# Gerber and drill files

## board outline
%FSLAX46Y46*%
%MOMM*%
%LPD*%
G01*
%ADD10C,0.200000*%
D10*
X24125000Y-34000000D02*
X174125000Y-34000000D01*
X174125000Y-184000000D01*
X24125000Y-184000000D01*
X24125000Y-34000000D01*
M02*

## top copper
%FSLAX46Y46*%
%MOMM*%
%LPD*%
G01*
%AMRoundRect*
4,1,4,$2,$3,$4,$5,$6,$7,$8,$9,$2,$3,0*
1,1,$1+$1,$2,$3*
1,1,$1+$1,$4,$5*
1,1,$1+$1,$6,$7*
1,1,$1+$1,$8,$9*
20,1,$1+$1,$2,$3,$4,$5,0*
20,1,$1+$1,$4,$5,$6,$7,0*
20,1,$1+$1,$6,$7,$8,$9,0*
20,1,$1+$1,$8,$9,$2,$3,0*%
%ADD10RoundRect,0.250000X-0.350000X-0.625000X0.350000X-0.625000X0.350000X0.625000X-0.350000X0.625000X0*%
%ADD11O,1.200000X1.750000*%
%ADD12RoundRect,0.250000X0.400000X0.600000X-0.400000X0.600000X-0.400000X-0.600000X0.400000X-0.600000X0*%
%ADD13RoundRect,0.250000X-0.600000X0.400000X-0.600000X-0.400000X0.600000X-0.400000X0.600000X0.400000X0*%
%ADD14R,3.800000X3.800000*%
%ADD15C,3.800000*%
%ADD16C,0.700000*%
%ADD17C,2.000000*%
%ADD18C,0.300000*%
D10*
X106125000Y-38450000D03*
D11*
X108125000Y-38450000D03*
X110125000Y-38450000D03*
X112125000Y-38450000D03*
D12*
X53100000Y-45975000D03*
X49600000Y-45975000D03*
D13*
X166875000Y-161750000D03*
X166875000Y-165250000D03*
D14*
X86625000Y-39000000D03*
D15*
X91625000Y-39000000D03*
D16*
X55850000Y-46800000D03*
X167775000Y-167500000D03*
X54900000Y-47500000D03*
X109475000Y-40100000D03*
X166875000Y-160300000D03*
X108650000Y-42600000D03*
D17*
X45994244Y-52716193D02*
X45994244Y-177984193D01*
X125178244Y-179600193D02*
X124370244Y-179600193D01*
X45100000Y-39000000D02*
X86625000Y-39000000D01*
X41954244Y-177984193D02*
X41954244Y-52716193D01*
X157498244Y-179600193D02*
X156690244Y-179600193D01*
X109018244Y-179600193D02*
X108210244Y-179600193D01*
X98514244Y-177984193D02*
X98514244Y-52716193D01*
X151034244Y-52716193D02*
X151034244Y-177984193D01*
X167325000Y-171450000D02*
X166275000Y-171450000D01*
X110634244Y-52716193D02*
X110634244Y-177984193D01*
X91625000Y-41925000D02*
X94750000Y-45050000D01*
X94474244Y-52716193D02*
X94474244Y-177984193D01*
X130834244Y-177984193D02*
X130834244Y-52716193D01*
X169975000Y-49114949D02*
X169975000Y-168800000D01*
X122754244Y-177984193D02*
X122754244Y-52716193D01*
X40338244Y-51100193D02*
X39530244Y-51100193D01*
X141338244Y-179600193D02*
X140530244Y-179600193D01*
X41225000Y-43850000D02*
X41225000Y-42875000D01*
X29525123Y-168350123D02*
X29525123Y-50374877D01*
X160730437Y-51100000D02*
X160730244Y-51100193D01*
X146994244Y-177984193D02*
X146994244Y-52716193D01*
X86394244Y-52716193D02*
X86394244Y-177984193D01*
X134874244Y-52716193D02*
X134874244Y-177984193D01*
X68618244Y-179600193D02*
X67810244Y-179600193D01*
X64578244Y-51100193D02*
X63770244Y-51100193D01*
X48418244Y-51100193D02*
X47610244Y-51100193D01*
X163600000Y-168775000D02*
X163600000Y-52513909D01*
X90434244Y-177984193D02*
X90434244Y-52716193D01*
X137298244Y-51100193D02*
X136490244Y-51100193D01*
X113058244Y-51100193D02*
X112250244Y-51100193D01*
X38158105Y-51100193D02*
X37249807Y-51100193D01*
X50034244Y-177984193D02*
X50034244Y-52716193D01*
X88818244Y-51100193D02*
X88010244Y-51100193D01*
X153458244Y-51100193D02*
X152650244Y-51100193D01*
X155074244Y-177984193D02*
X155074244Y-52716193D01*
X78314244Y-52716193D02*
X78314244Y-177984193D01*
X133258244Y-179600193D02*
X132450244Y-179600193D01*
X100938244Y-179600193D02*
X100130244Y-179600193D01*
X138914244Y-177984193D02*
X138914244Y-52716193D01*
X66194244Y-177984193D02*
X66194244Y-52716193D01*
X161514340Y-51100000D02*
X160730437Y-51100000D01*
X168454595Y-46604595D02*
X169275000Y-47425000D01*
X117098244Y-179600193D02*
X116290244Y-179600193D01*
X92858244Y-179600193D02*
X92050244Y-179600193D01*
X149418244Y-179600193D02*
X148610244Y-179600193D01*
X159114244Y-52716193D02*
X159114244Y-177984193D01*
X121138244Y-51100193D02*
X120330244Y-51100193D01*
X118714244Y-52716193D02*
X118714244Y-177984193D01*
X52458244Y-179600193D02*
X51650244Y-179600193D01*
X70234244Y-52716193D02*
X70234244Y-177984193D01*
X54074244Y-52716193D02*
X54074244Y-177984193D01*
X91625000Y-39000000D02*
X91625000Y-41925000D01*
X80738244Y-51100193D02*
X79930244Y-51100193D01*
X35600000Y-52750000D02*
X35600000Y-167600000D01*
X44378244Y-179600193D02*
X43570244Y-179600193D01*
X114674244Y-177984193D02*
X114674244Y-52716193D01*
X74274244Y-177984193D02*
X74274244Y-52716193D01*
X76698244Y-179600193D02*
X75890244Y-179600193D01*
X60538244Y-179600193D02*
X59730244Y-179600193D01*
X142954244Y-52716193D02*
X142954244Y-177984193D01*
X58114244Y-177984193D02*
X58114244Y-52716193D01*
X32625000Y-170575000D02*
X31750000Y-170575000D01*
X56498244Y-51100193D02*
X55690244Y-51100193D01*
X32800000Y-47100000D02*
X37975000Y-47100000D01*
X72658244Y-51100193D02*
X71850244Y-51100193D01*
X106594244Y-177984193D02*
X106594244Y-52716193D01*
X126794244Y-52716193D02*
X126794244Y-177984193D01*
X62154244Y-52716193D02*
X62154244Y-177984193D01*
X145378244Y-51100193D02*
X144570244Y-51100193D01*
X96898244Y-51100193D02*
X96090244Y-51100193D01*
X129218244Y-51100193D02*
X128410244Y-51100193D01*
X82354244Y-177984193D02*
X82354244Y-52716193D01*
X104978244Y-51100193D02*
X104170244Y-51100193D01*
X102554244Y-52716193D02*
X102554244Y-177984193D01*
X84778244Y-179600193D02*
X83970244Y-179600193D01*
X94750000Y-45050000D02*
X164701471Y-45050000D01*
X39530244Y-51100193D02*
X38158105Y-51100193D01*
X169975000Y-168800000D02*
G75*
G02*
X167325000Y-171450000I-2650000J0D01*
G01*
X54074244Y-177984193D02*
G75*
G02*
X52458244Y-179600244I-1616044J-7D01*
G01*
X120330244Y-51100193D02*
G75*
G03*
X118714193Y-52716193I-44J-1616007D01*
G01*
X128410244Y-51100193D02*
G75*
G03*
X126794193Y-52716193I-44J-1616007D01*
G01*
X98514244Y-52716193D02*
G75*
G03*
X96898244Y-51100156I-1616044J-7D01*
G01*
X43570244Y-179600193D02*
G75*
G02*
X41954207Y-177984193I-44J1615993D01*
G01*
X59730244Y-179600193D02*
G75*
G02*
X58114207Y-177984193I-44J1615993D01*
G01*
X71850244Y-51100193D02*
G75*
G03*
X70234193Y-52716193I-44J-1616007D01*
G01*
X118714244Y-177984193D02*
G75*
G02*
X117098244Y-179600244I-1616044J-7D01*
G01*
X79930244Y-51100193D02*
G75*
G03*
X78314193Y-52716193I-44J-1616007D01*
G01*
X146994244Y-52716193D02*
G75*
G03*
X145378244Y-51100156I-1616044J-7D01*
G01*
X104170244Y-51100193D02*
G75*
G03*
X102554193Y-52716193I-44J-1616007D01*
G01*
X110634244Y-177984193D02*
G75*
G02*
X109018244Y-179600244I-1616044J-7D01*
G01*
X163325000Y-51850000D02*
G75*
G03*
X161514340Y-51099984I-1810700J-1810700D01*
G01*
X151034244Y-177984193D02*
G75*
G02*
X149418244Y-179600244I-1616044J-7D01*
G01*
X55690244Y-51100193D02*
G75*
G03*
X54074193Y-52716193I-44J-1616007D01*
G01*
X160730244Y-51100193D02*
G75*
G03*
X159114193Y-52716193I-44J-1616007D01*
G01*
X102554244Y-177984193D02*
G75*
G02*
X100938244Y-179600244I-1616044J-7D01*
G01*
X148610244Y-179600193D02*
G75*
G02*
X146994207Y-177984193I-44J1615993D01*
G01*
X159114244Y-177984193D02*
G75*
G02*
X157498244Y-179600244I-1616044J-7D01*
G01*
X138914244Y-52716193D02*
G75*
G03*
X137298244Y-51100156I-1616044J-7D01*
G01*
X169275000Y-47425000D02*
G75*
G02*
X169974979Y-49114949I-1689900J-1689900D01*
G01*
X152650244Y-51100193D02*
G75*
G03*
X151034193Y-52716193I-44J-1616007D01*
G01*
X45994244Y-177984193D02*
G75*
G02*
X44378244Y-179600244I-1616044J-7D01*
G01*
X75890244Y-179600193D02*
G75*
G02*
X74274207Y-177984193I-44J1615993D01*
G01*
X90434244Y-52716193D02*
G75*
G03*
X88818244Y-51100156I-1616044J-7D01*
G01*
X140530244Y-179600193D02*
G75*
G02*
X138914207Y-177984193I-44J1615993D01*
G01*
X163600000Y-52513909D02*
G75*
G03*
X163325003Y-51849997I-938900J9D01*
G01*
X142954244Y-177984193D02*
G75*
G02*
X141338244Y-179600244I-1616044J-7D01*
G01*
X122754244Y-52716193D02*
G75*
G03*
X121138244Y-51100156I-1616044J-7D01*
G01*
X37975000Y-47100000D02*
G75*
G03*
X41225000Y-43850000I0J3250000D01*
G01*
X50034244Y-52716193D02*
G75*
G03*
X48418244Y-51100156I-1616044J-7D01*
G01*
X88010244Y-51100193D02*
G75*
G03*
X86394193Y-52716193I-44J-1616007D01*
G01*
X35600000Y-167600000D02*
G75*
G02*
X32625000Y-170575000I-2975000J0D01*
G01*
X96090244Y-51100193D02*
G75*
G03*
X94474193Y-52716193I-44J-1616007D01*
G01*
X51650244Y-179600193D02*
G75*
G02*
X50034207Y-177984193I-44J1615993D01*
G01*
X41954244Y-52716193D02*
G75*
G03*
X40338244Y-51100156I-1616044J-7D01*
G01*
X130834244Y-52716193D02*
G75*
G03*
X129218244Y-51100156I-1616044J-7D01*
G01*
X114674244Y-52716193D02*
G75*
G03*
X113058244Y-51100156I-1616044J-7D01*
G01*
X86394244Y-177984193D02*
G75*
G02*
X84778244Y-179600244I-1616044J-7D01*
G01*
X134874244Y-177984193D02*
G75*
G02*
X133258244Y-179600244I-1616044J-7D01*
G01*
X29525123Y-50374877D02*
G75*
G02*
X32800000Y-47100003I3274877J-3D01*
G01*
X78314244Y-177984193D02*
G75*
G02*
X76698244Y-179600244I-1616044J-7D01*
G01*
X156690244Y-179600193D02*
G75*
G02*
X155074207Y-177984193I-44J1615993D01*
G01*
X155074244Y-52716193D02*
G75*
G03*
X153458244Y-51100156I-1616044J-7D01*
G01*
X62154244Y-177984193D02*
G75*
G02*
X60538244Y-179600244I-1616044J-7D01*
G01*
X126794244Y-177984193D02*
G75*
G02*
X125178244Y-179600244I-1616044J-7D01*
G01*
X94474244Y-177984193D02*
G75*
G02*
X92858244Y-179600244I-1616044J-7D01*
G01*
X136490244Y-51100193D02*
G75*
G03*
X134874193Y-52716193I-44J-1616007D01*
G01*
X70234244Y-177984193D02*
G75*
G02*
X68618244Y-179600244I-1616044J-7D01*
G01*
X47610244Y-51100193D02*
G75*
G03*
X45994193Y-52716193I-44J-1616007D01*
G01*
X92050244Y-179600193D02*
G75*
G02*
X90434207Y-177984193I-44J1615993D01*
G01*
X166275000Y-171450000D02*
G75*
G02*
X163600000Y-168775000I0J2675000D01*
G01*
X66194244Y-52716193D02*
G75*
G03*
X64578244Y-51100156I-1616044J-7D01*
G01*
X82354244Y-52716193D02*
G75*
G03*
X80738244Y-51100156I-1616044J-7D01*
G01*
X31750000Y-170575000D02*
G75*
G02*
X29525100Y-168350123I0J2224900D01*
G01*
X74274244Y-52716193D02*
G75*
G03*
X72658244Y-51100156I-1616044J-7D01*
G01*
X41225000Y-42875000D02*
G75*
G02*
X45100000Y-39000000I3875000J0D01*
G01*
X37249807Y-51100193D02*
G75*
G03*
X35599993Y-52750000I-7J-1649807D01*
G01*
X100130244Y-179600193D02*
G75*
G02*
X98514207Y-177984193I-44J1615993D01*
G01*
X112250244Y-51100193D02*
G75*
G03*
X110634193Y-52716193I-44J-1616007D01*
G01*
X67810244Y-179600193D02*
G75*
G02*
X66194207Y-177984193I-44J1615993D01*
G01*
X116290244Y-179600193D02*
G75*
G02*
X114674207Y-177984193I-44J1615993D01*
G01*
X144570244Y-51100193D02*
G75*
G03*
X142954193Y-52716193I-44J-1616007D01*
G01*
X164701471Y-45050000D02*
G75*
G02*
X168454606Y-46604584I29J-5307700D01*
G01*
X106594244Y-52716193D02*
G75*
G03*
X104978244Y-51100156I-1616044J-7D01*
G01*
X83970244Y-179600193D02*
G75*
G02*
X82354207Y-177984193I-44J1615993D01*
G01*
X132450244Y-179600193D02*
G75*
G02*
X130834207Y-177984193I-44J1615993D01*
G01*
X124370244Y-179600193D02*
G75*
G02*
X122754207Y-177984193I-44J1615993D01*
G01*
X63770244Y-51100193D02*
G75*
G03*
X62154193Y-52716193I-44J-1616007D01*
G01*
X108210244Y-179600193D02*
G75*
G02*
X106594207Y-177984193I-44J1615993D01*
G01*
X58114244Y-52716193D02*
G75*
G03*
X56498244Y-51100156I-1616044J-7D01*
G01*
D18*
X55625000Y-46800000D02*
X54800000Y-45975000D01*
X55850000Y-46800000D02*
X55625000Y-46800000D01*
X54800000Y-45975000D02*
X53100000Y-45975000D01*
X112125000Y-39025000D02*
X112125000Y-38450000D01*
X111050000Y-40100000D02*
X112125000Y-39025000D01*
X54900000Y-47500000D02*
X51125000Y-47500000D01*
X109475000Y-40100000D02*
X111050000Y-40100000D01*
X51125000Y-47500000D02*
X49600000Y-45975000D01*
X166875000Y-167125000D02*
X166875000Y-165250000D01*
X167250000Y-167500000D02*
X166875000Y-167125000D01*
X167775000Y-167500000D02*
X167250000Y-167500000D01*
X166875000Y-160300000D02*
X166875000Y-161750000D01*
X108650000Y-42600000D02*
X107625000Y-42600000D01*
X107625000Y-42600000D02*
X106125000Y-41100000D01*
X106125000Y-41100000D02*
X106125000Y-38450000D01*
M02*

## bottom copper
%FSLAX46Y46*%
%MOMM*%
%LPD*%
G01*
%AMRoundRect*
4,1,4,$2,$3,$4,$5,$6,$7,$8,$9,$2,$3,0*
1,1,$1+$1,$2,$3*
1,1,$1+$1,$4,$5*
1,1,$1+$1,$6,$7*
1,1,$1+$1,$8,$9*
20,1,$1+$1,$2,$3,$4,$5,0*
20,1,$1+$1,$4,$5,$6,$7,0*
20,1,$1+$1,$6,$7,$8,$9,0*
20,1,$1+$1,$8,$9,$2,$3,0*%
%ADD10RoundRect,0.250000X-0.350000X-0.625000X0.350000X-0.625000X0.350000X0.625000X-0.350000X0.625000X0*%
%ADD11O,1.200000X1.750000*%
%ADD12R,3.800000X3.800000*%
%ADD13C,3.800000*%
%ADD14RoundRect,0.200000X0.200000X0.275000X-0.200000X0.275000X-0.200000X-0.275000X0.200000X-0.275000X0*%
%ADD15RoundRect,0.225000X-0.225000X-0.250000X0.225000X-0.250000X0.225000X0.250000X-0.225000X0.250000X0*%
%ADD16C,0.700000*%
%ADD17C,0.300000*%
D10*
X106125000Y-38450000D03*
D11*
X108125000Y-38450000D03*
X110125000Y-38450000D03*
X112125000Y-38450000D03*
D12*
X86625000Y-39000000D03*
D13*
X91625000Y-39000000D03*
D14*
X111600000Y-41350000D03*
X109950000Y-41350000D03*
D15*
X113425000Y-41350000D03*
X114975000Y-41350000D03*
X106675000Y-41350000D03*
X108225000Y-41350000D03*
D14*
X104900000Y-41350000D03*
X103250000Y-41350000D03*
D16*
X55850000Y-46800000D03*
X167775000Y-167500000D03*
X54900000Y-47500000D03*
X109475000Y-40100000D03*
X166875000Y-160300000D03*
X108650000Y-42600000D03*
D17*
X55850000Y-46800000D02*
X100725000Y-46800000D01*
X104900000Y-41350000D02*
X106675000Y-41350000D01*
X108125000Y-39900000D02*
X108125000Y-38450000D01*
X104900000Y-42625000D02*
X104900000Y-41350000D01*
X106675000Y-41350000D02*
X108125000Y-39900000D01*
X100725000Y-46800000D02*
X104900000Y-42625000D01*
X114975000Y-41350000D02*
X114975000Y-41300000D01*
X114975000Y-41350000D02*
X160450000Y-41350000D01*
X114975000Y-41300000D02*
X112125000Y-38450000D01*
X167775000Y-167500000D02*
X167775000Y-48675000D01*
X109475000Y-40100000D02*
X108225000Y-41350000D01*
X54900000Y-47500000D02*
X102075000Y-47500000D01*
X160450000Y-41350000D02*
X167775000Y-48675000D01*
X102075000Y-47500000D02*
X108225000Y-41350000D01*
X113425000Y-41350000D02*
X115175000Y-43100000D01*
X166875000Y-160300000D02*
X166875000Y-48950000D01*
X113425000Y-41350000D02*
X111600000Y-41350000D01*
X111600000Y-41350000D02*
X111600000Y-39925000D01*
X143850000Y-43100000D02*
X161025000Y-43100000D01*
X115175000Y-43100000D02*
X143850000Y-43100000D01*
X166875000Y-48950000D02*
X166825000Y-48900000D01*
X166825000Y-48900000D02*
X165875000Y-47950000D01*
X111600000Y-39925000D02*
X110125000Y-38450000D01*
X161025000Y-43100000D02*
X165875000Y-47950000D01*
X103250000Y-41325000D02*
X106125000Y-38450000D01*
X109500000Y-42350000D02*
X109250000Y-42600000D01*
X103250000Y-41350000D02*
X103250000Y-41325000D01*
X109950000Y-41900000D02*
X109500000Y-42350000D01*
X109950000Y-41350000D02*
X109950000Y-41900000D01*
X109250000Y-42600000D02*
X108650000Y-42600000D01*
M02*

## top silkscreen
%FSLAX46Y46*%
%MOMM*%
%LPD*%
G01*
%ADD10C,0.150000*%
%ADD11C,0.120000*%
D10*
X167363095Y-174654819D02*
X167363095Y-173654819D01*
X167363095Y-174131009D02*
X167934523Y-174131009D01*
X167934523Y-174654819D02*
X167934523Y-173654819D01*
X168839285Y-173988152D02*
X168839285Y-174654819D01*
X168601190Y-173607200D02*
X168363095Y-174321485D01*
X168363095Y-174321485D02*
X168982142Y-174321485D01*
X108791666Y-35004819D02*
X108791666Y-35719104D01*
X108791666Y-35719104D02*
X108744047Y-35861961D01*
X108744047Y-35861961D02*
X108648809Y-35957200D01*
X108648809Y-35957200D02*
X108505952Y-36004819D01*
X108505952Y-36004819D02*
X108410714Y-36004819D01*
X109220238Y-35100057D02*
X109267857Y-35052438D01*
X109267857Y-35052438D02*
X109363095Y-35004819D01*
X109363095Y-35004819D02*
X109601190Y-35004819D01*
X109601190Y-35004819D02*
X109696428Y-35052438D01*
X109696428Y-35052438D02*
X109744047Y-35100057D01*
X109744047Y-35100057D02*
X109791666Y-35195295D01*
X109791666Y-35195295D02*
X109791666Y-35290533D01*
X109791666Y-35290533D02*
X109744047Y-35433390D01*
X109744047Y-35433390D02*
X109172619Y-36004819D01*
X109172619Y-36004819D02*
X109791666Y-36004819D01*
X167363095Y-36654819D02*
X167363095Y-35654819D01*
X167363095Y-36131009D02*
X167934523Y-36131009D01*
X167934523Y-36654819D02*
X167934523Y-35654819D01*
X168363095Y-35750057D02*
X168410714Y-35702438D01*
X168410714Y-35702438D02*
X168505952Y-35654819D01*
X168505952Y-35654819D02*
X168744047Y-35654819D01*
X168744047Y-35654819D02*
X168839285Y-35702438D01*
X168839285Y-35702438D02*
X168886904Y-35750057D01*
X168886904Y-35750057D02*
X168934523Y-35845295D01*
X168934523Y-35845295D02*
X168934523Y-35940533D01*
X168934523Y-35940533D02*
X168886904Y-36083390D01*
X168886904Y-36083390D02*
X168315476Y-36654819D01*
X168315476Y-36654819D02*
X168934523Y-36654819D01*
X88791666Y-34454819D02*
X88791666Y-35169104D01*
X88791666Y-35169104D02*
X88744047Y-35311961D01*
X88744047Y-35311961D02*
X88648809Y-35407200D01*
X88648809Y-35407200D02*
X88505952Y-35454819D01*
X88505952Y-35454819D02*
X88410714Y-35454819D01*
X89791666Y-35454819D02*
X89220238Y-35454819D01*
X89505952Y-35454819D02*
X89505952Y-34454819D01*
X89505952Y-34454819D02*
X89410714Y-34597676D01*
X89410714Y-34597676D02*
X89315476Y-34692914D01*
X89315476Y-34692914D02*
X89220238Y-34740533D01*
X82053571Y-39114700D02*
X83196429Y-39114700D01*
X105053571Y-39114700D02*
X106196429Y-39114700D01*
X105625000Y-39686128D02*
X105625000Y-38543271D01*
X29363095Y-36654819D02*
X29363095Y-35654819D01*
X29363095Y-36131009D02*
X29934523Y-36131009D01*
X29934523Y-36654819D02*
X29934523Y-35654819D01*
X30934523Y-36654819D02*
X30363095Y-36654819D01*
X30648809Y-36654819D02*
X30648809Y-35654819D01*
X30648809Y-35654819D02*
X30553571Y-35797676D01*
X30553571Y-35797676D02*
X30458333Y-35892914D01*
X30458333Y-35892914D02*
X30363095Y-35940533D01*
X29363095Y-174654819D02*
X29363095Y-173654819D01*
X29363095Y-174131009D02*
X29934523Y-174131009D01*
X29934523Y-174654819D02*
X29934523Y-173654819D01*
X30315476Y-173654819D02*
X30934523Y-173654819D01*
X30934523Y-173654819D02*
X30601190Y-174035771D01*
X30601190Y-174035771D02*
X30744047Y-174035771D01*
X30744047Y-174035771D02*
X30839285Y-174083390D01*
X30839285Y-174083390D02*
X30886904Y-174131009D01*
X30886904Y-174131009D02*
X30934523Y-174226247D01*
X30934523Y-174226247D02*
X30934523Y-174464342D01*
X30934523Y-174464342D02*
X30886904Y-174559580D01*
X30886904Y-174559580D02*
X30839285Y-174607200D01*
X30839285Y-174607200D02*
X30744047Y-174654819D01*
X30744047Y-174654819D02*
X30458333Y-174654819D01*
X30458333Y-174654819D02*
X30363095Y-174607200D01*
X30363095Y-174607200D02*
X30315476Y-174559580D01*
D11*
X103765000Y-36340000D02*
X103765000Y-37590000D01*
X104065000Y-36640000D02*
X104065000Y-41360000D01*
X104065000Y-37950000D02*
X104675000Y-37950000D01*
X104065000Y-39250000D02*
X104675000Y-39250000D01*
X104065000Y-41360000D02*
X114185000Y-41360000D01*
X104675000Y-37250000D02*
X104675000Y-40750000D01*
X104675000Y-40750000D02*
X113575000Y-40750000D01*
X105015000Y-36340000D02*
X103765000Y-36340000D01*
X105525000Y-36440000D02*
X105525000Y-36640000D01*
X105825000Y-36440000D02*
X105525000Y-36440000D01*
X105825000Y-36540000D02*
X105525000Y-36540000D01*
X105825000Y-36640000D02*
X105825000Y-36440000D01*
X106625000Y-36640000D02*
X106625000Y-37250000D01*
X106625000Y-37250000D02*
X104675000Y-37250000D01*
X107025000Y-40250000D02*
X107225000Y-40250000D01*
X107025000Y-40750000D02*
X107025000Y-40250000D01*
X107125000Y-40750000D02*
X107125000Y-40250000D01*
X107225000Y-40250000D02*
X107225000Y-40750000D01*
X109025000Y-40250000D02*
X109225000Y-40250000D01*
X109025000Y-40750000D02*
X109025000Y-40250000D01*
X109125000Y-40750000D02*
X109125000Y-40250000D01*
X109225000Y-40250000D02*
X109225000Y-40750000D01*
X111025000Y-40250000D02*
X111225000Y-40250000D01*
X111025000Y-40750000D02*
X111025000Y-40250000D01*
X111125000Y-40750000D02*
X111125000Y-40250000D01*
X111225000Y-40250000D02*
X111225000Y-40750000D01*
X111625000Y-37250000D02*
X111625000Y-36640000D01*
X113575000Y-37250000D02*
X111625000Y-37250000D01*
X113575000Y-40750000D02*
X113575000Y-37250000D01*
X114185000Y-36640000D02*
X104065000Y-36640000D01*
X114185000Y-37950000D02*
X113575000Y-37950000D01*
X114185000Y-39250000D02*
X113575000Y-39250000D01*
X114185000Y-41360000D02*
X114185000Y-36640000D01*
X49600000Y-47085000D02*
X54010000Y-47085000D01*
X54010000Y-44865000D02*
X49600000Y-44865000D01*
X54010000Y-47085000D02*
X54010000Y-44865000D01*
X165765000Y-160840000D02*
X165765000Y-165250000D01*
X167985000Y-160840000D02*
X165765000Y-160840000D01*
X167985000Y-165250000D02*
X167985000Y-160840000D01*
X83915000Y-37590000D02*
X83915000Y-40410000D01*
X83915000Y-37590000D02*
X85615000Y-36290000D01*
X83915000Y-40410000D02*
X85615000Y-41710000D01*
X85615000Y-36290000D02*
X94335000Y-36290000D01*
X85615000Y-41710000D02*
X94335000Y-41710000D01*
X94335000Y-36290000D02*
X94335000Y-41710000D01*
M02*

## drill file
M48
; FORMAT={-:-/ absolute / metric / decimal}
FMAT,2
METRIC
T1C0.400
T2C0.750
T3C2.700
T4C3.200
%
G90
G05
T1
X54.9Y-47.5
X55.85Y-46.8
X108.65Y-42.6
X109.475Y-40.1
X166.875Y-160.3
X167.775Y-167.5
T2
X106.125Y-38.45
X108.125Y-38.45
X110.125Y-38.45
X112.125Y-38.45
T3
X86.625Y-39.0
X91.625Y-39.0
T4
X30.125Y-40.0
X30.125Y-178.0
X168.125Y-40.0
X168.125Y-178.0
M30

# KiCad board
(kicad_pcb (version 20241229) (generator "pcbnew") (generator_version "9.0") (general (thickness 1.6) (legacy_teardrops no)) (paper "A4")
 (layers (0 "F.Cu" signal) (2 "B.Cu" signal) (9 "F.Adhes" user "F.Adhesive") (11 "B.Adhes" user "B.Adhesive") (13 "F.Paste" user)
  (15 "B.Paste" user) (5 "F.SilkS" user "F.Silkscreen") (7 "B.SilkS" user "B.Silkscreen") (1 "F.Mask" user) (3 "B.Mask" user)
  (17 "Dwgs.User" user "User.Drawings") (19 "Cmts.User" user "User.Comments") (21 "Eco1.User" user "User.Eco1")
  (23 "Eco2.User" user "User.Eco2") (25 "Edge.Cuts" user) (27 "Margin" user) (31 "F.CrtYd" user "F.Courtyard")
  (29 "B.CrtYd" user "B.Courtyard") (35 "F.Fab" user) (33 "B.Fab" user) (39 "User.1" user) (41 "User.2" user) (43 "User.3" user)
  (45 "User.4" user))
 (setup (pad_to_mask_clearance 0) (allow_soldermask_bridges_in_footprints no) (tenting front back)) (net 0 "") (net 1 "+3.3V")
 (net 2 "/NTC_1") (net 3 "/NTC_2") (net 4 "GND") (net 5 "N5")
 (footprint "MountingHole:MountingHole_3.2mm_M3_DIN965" (layer "F.Cu") (at 168.125 178)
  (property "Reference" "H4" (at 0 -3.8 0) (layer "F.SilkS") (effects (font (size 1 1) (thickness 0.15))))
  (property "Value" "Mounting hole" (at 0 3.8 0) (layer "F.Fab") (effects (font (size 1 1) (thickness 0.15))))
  (pad "" np_thru_hole circle (at 0 0) (size 3.2 3.2) (drill 3.2) (layers "*.Cu" "*.Mask")))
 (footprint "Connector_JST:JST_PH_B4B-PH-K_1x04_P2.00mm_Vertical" (layer "F.Cu") (at 106.125 38.45)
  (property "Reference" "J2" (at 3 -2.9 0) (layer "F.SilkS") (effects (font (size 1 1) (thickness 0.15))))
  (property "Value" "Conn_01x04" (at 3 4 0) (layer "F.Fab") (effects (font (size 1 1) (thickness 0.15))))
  (fp_line (start -2.36 -2.11) (end -2.36 -0.86) (stroke (width 0.12) (type solid)) (layer "F.SilkS"))
  (fp_line (start -2.06 -1.81) (end -2.06 2.91) (stroke (width 0.12) (type solid)) (layer "F.SilkS"))
  (fp_line (start -2.06 -0.5) (end -1.45 -0.5) (stroke (width 0.12) (type solid)) (layer "F.SilkS"))
  (fp_line (start -2.06 0.8) (end -1.45 0.8) (stroke (width 0.12) (type solid)) (layer "F.SilkS"))
  (fp_line (start -2.06 2.91) (end 8.06 2.91) (stroke (width 0.12) (type solid)) (layer "F.SilkS"))
  (fp_line (start -1.45 -1.2) (end -1.45 2.3) (stroke (width 0.12) (type solid)) (layer "F.SilkS"))
  (fp_line (start -1.45 2.3) (end 7.45 2.3) (stroke (width 0.12) (type solid)) (layer "F.SilkS"))
  (fp_line (start -1.11 -2.11) (end -2.36 -2.11) (stroke (width 0.12) (type solid)) (layer "F.SilkS"))
  (fp_line (start -0.6 -2.01) (end -0.6 -1.81) (stroke (width 0.12) (type solid)) (layer "F.SilkS"))
  (fp_line (start -0.3 -2.01) (end -0.6 -2.01) (stroke (width 0.12) (type solid)) (layer "F.SilkS"))
  (fp_line (start -0.3 -1.91) (end -0.6 -1.91) (stroke (width 0.12) (type solid)) (layer "F.SilkS"))
  (fp_line (start -0.3 -1.81) (end -0.3 -2.01) (stroke (width 0.12) (type solid)) (layer "F.SilkS"))
  (fp_line (start 0.5 -1.81) (end 0.5 -1.2) (stroke (width 0.12) (type solid)) (layer "F.SilkS"))
  (fp_line (start 0.5 -1.2) (end -1.45 -1.2) (stroke (width 0.12) (type solid)) (layer "F.SilkS"))
  (fp_line (start 0.9 1.8) (end 1.1 1.8) (stroke (width 0.12) (type solid)) (layer "F.SilkS"))
  (fp_line (start 0.9 2.3) (end 0.9 1.8) (stroke (width 0.12) (type solid)) (layer "F.SilkS"))
  (fp_line (start 1 2.3) (end 1 1.8) (stroke (width 0.12) (type solid)) (layer "F.SilkS"))
  (fp_line (start 1.1 1.8) (end 1.1 2.3) (stroke (width 0.12) (type solid)) (layer "F.SilkS"))
  (fp_line (start 2.9 1.8) (end 3.1 1.8) (stroke (width 0.12) (type solid)) (layer "F.SilkS"))
  (fp_line (start 2.9 2.3) (end 2.9 1.8) (stroke (width 0.12) (type solid)) (layer "F.SilkS"))
  (fp_line (start 3 2.3) (end 3 1.8) (stroke (width 0.12) (type solid)) (layer "F.SilkS"))
  (fp_line (start 3.1 1.8) (end 3.1 2.3) (stroke (width 0.12) (type solid)) (layer "F.SilkS"))
  (fp_line (start 4.9 1.8) (end 5.1 1.8) (stroke (width 0.12) (type solid)) (layer "F.SilkS"))
  (fp_line (start 4.9 2.3) (end 4.9 1.8) (stroke (width 0.12) (type solid)) (layer "F.SilkS"))
  (fp_line (start 5 2.3) (end 5 1.8) (stroke (width 0.12) (type solid)) (layer "F.SilkS"))
  (fp_line (start 5.1 1.8) (end 5.1 2.3) (stroke (width 0.12) (type solid)) (layer "F.SilkS"))
  (fp_line (start 5.5 -1.2) (end 5.5 -1.81) (stroke (width 0.12) (type solid)) (layer "F.SilkS"))
  (fp_line (start 7.45 -1.2) (end 5.5 -1.2) (stroke (width 0.12) (type solid)) (layer "F.SilkS"))
  (fp_line (start 7.45 2.3) (end 7.45 -1.2) (stroke (width 0.12) (type solid)) (layer "F.SilkS"))
  (fp_line (start 8.06 -1.81) (end -2.06 -1.81) (stroke (width 0.12) (type solid)) (layer "F.SilkS"))
  (fp_line (start 8.06 -0.5) (end 7.45 -0.5) (stroke (width 0.12) (type solid)) (layer "F.SilkS"))
  (fp_line (start 8.06 0.8) (end 7.45 0.8) (stroke (width 0.12) (type solid)) (layer "F.SilkS"))
  (fp_line (start 8.06 2.91) (end 8.06 -1.81) (stroke (width 0.12) (type solid)) (layer "F.SilkS"))
  (pad "1" thru_hole roundrect (at 0 0) (size 1.2 1.75) (drill 0.75) (layers "*.Cu" "*.Mask") (remove_unused_layers no)
   (roundrect_rratio 0.208333) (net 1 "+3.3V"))
  (pad "2" thru_hole oval (at 2 0) (size 1.2 1.75) (drill 0.75) (layers "*.Cu" "*.Mask") (remove_unused_layers no) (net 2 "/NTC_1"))
  (pad "3" thru_hole oval (at 4 0) (size 1.2 1.75) (drill 0.75) (layers "*.Cu" "*.Mask") (remove_unused_layers no) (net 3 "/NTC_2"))
  (pad "4" thru_hole oval (at 6 0) (size 1.2 1.75) (drill 0.75) (layers "*.Cu" "*.Mask") (remove_unused_layers no) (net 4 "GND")))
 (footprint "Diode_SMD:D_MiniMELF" (layer "F.Cu") (at 51.35 45.975 180)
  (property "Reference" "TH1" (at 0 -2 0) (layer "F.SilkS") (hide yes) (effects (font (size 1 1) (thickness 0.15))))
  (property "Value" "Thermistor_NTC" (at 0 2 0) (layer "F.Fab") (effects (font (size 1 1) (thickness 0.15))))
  (fp_line (start 1.75 -1.11) (end -2.66 -1.11) (stroke (width 0.12) (type solid)) (layer "F.SilkS"))
  (fp_line (start -2.66 1.11) (end 1.75 1.11) (stroke (width 0.12) (type solid)) (layer "F.SilkS"))
  (fp_line (start -2.66 -1.11) (end -2.66 1.11) (stroke (width 0.12) (type solid)) (layer "F.SilkS"))
  (pad "1" smd roundrect (at -1.75 0 180) (size 1.3 1.7) (layers "F.Cu" "F.Mask" "F.Paste") (roundrect_rratio 0.1923076923) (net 2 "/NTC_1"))
  (pad "2" smd roundrect (at 1.75 0 180) (size 1.3 1.7) (layers "F.Cu" "F.Mask" "F.Paste") (roundrect_rratio 0.1923076923) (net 4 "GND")))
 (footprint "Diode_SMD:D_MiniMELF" (layer "F.Cu") (at 166.875 163.5 -90)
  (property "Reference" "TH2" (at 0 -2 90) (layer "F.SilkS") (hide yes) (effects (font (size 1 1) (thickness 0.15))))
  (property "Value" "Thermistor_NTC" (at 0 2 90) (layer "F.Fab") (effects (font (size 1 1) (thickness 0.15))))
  (fp_line (start -2.66 1.11) (end 1.75 1.11) (stroke (width 0.12) (type solid)) (layer "F.SilkS"))
  (fp_line (start -2.66 -1.11) (end -2.66 1.11) (stroke (width 0.12) (type solid)) (layer "F.SilkS"))
  (fp_line (start 1.75 -1.11) (end -2.66 -1.11) (stroke (width 0.12) (type solid)) (layer "F.SilkS"))
  (pad "1" smd roundrect (at -1.75 0 270) (size 1.3 1.7) (layers "F.Cu" "F.Mask" "F.Paste") (roundrect_rratio 0.1923076923) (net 3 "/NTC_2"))
  (pad "2" smd roundrect (at 1.75 0 270) (size 1.3 1.7) (layers "F.Cu" "F.Mask" "F.Paste") (roundrect_rratio 0.1923076923) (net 4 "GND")))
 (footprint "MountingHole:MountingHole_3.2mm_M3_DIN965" (layer "F.Cu") (at 168.125 40)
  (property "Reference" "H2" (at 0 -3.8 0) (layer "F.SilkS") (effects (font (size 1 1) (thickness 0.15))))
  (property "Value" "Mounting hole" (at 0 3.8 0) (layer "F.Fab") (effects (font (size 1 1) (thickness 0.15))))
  (pad "" np_thru_hole circle (at 0 0) (size 3.2 3.2) (drill 3.2) (layers "*.Cu" "*.Mask")))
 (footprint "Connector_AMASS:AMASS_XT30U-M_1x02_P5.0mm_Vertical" (layer "F.Cu") (at 86.625 39)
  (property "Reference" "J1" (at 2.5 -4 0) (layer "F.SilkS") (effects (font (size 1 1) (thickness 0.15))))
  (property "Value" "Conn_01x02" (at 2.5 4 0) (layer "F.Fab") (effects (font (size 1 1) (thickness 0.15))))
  (fp_line (start -2.71 -1.41) (end -2.71 1.41) (stroke (width 0.12) (type solid)) (layer "F.SilkS"))
  (fp_line (start -2.71 -1.41) (end -1.01 -2.71) (stroke (width 0.12) (type solid)) (layer "F.SilkS"))
  (fp_line (start -2.71 1.41) (end -1.01 2.71) (stroke (width 0.12) (type solid)) (layer "F.SilkS"))
  (fp_line (start -1.01 -2.71) (end 7.71 -2.71) (stroke (width 0.12) (type solid)) (layer "F.SilkS"))
  (fp_line (start -1.01 2.71) (end 7.71 2.71) (stroke (width 0.12) (type solid)) (layer "F.SilkS"))
  (fp_line (start 7.71 -2.71) (end 7.71 2.71) (stroke (width 0.12) (type solid)) (layer "F.SilkS"))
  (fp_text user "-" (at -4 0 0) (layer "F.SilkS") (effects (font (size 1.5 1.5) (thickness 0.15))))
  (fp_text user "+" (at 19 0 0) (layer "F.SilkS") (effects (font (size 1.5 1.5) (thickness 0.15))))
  (pad "1" thru_hole rect (at 0 0) (size 3.8 3.8) (drill 2.7) (layers "*.Cu" "*.Mask") (remove_unused_layers no) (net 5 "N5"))
  (pad "2" thru_hole circle (at 5 0) (size 3.8 3.8) (drill 2.7) (layers "*.Cu" "*.Mask") (remove_unused_layers no) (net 5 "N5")))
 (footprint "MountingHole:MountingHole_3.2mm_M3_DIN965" (layer "F.Cu") (at 30.125 40)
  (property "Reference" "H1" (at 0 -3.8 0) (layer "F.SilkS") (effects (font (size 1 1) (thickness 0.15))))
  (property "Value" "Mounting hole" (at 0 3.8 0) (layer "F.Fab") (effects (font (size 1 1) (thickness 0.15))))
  (pad "" np_thru_hole circle (at 0 0) (size 3.2 3.2) (drill 3.2) (layers "*.Cu" "*.Mask")))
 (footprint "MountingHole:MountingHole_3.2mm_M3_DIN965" (layer "F.Cu") (at 30.125 178)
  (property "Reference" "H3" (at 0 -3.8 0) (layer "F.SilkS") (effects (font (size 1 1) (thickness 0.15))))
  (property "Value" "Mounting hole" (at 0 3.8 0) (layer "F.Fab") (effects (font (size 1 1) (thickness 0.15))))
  (pad "" np_thru_hole circle (at 0 0) (size 3.2 3.2) (drill 3.2) (layers "*.Cu" "*.Mask")))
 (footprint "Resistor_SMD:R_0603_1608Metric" (layer "B.Cu") (at 110.775 41.35 180)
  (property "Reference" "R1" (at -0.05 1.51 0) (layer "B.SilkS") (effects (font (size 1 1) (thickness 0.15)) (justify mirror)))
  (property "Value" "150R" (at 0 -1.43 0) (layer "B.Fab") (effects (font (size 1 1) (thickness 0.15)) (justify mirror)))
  (pad "1" smd roundrect (at -0.825 0 180) (size 0.8 0.95) (layers "B.Cu" "B.Mask" "B.Paste") (roundrect_rratio 0.25) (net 3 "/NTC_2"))
  (pad "2" smd roundrect (at 0.825 0 180) (size 0.8 0.95) (layers "B.Cu" "B.Mask" "B.Paste") (roundrect_rratio 0.25) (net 1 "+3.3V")))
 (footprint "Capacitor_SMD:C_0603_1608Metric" (layer "B.Cu") (at 114.2 41.35)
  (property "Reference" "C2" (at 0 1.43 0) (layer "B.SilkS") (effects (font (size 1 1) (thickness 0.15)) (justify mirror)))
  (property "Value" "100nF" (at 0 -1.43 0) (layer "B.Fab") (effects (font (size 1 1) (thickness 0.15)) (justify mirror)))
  (pad "1" smd roundrect (at -0.775 0) (size 0.9 0.95) (layers "B.Cu" "B.Mask" "B.Paste") (roundrect_rratio 0.25) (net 3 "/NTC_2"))
  (pad "2" smd roundrect (at 0.775 0) (size 0.9 0.95) (layers "B.Cu" "B.Mask" "B.Paste") (roundrect_rratio 0.25) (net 4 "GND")))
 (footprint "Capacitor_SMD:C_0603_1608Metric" (layer "B.Cu") (at 107.45 41.35)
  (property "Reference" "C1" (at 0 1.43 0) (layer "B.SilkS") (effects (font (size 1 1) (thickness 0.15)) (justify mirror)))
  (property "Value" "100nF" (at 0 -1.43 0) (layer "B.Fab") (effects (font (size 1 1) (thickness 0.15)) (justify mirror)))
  (pad "1" smd roundrect (at -0.775 0) (size 0.9 0.95) (layers "B.Cu" "B.Mask" "B.Paste") (roundrect_rratio 0.25) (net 2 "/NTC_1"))
  (pad "2" smd roundrect (at 0.775 0) (size 0.9 0.95) (layers "B.Cu" "B.Mask" "B.Paste") (roundrect_rratio 0.25) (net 4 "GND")))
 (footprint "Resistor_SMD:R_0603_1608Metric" (layer "B.Cu") (at 104.075 41.35 180)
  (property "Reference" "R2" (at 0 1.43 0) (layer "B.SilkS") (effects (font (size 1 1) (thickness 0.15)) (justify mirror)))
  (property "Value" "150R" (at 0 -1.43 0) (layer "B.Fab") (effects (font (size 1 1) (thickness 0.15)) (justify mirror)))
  (pad "1" smd roundrect (at -0.825 0 180) (size 0.8 0.95) (layers "B.Cu" "B.Mask" "B.Paste") (roundrect_rratio 0.25) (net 2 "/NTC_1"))
  (pad "2" smd roundrect (at 0.825 0 180) (size 0.8 0.95) (layers "B.Cu" "B.Mask" "B.Paste") (roundrect_rratio 0.25) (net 1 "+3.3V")))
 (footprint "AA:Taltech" (layer "B.Cu") (at 156.95 79.6 180)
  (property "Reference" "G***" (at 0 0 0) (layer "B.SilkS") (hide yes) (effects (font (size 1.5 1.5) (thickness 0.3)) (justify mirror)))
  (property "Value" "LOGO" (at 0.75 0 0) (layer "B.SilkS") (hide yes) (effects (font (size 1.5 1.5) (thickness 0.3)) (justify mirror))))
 (gr_rect (start 24.125 34) (end 174.125 184) (stroke (width 0.2) (type solid)) (fill no) (layer "Edge.Cuts"))
 (segment (start 45.994244 52.716193) (end 45.994244 177.984193) (width 2) (layer "F.Cu") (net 5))
 (segment (start 125.178244 179.600193) (end 124.370244 179.600193) (width 2) (layer "F.Cu") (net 5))
 (segment (start 45.1 39) (end 86.625 39) (width 2) (layer "F.Cu") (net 5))
 (segment (start 41.954244 177.984193) (end 41.954244 52.716193) (width 2) (layer "F.Cu") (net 5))
 (segment (start 157.498244 179.600193) (end 156.690244 179.600193) (width 2) (layer "F.Cu") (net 5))
 (segment (start 109.018244 179.600193) (end 108.210244 179.600193) (width 2) (layer "F.Cu") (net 5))
 (segment (start 98.514244 177.984193) (end 98.514244 52.716193) (width 2) (layer "F.Cu") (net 5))
 (segment (start 151.034244 52.716193) (end 151.034244 177.984193) (width 2) (layer "F.Cu") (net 5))
 (segment (start 167.325 171.45) (end 166.275 171.45) (width 2) (layer "F.Cu") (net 5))
 (segment (start 110.634244 52.716193) (end 110.634244 177.984193) (width 2) (layer "F.Cu") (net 5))
 (segment (start 91.625 41.925) (end 94.75 45.05) (width 2) (layer "F.Cu") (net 5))
 (segment (start 94.474244 52.716193) (end 94.474244 177.984193) (width 2) (layer "F.Cu") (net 5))
 (segment (start 130.834244 177.984193) (end 130.834244 52.716193) (width 2) (layer "F.Cu") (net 5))
 (segment (start 169.975 49.114949) (end 169.975 168.8) (width 2) (layer "F.Cu") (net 5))
 (segment (start 122.754244 177.984193) (end 122.754244 52.716193) (width 2) (layer "F.Cu") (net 5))
 (segment (start 40.338244 51.100193) (end 39.530244 51.100193) (width 2) (layer "F.Cu") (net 5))
 (segment (start 141.338244 179.600193) (end 140.530244 179.600193) (width 2) (layer "F.Cu") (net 5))
 (segment (start 41.225 43.85) (end 41.225 42.875) (width 2) (layer "F.Cu") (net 5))
 (segment (start 29.525123 168.350123) (end 29.525123 50.374877) (width 2) (layer "F.Cu") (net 5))
 (segment (start 160.730437 51.1) (end 160.730244 51.100193) (width 2) (layer "F.Cu") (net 5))
 (segment (start 146.994244 177.984193) (end 146.994244 52.716193) (width 2) (layer "F.Cu") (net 5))
 (segment (start 86.394244 52.716193) (end 86.394244 177.984193) (width 2) (layer "F.Cu") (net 5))
 (segment (start 134.874244 52.716193) (end 134.874244 177.984193) (width 2) (layer "F.Cu") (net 5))
 (segment (start 68.618244 179.600193) (end 67.810244 179.600193) (width 2) (layer "F.Cu") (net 5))
 (segment (start 64.578244 51.100193) (end 63.770244 51.100193) (width 2) (layer "F.Cu") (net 5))
 (segment (start 48.418244 51.100193) (end 47.610244 51.100193) (width 2) (layer "F.Cu") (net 5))
 (segment (start 163.6 168.775) (end 163.6 52.513909) (width 2) (layer "F.Cu") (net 5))
 (segment (start 90.434244 177.984193) (end 90.434244 52.716193) (width 2) (layer "F.Cu") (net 5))
 (segment (start 137.298244 51.100193) (end 136.490244 51.100193) (width 2) (layer "F.Cu") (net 5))
 (segment (start 113.058244 51.100193) (end 112.250244 51.100193) (width 2) (layer "F.Cu") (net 5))
 (segment (start 38.158105 51.100193) (end 37.249807 51.100193) (width 2) (layer "F.Cu") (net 5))
 (segment (start 50.034244 177.984193) (end 50.034244 52.716193) (width 2) (layer "F.Cu") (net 5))
 (segment (start 88.818244 51.100193) (end 88.010244 51.100193) (width 2) (layer "F.Cu") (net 5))
 (segment (start 153.458244 51.100193) (end 152.650244 51.100193) (width 2) (layer "F.Cu") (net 5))
 (segment (start 155.074244 177.984193) (end 155.074244 52.716193) (width 2) (layer "F.Cu") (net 5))
 (segment (start 78.314244 52.716193) (end 78.314244 177.984193) (width 2) (layer "F.Cu") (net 5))
 (segment (start 133.258244 179.600193) (end 132.450244 179.600193) (width 2) (layer "F.Cu") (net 5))
 (segment (start 100.938244 179.600193) (end 100.130244 179.600193) (width 2) (layer "F.Cu") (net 5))
 (segment (start 138.914244 177.984193) (end 138.914244 52.716193) (width 2) (layer "F.Cu") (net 5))
 (segment (start 66.194244 177.984193) (end 66.194244 52.716193) (width 2) (layer "F.Cu") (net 5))
 (segment (start 161.51434 51.1) (end 160.730437 51.1) (width 2) (layer "F.Cu") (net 5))
 (segment (start 168.454595 46.604595) (end 169.275 47.425) (width 2) (layer "F.Cu") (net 5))
 (segment (start 117.098244 179.600193) (end 116.290244 179.600193) (width 2) (layer "F.Cu") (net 5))
 (segment (start 92.858244 179.600193) (end 92.050244 179.600193) (width 2) (layer "F.Cu") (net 5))
 (segment (start 149.418244 179.600193) (end 148.610244 179.600193) (width 2) (layer "F.Cu") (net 5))
 (segment (start 159.114244 52.716193) (end 159.114244 177.984193) (width 2) (layer "F.Cu") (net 5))
 (segment (start 121.138244 51.100193) (end 120.330244 51.100193) (width 2) (layer "F.Cu") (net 5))
 (segment (start 118.714244 52.716193) (end 118.714244 177.984193) (width 2) (layer "F.Cu") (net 5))
 (segment (start 52.458244 179.600193) (end 51.650244 179.600193) (width 2) (layer "F.Cu") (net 5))
 (segment (start 70.234244 52.716193) (end 70.234244 177.984193) (width 2) (layer "F.Cu") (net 5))
 (segment (start 54.074244 52.716193) (end 54.074244 177.984193) (width 2) (layer "F.Cu") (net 5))
 (segment (start 91.625 39) (end 91.625 41.925) (width 2) (layer "F.Cu") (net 5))
 (segment (start 80.738244 51.100193) (end 79.930244 51.100193) (width 2) (layer "F.Cu") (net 5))
 (segment (start 35.6 52.75) (end 35.6 167.6) (width 2) (layer "F.Cu") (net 5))
 (segment (start 44.378244 179.600193) (end 43.570244 179.600193) (width 2) (layer "F.Cu") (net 5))
 (segment (start 114.674244 177.984193) (end 114.674244 52.716193) (width 2) (layer "F.Cu") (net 5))
 (segment (start 74.274244 177.984193) (end 74.274244 52.716193) (width 2) (layer "F.Cu") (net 5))
 (segment (start 76.698244 179.600193) (end 75.890244 179.600193) (width 2) (layer "F.Cu") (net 5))
 (segment (start 60.538244 179.600193) (end 59.730244 179.600193) (width 2) (layer "F.Cu") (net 5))
 (segment (start 142.954244 52.716193) (end 142.954244 177.984193) (width 2) (layer "F.Cu") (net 5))
 (segment (start 58.114244 177.984193) (end 58.114244 52.716193) (width 2) (layer "F.Cu") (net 5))
 (segment (start 32.625 170.575) (end 31.75 170.575) (width 2) (layer "F.Cu") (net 5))
 (segment (start 56.498244 51.100193) (end 55.690244 51.100193) (width 2) (layer "F.Cu") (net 5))
 (segment (start 32.8 47.1) (end 37.975 47.1) (width 2) (layer "F.Cu") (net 5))
 (segment (start 72.658244 51.100193) (end 71.850244 51.100193) (width 2) (layer "F.Cu") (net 5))
 (segment (start 106.594244 177.984193) (end 106.594244 52.716193) (width 2) (layer "F.Cu") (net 5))
 (segment (start 126.794244 52.716193) (end 126.794244 177.984193) (width 2) (layer "F.Cu") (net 5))
 (segment (start 62.154244 52.716193) (end 62.154244 177.984193) (width 2) (layer "F.Cu") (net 5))
 (segment (start 145.378244 51.100193) (end 144.570244 51.100193) (width 2) (layer "F.Cu") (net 5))
 (segment (start 96.898244 51.100193) (end 96.090244 51.100193) (width 2) (layer "F.Cu") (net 5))
 (segment (start 129.218244 51.100193) (end 128.410244 51.100193) (width 2) (layer "F.Cu") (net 5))
 (segment (start 82.354244 177.984193) (end 82.354244 52.716193) (width 2) (layer "F.Cu") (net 5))
 (segment (start 104.978244 51.100193) (end 104.170244 51.100193) (width 2) (layer "F.Cu") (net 5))
 (segment (start 102.554244 52.716193) (end 102.554244 177.984193) (width 2) (layer "F.Cu") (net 5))
 (segment (start 84.778244 179.600193) (end 83.970244 179.600193) (width 2) (layer "F.Cu") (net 5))
 (segment (start 94.75 45.05) (end 164.701471 45.05) (width 2) (layer "F.Cu") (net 5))
 (segment (start 39.530244 51.100193) (end 38.158105 51.100193) (width 2) (layer "F.Cu") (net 5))
 (arc (start 169.975 168.8) (mid 169.198833 170.673833) (end 167.325 171.45) (width 2) (layer "F.Cu") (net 5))
 (arc (start 54.074244 177.984193) (mid 53.600929 179.126878) (end 52.458244 179.600193) (width 2) (layer "F.Cu") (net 5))
 (arc (start 120.330244 51.100193) (mid 119.187559 51.573508) (end 118.714244 52.716193) (width 2) (layer "F.Cu") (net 5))
 (arc (start 128.410244 51.100193) (mid 127.267559 51.573508) (end 126.794244 52.716193) (width 2) (layer "F.Cu") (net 5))
 (arc (start 98.514244 52.716193) (mid 98.040929 51.573508) (end 96.898244 51.100193) (width 2) (layer "F.Cu") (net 5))
 (arc (start 43.570244 179.600193) (mid 42.427559 179.126878) (end 41.954244 177.984193) (width 2) (layer "F.Cu") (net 5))
 (arc (start 59.730244 179.600193) (mid 58.587559 179.126878) (end 58.114244 177.984193) (width 2) (layer "F.Cu") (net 5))
 (arc (start 71.850244 51.100193) (mid 70.707559 51.573508) (end 70.234244 52.716193) (width 2) (layer "F.Cu") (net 5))
 (arc (start 118.714244 177.984193) (mid 118.240929 179.126878) (end 117.098244 179.600193) (width 2) (layer "F.Cu") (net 5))
 (arc (start 79.930244 51.100193) (mid 78.787559 51.573508) (end 78.314244 52.716193) (width 2) (layer "F.Cu") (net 5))
 (arc (start 146.994244 52.716193) (mid 146.520929 51.573508) (end 145.378244 51.100193) (width 2) (layer "F.Cu") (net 5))
 (arc (start 104.170244 51.100193) (mid 103.027559 51.573508) (end 102.554244 52.716193) (width 2) (layer "F.Cu") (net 5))
 (arc (start 110.634244 177.984193) (mid 110.160929 179.126878) (end 109.018244 179.600193) (width 2) (layer "F.Cu") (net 5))
 (arc (start 163.325 51.85) (mid 162.494262 51.294918) (end 161.51434 51.1) (width 2) (layer "F.Cu") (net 5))
 (arc (start 151.034244 177.984193) (mid 150.560929 179.126878) (end 149.418244 179.600193) (width 2) (layer "F.Cu") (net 5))
 (arc (start 55.690244 51.100193) (mid 54.547559 51.573508) (end 54.074244 52.716193) (width 2) (layer "F.Cu") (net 5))
 (arc (start 160.730244 51.100193) (mid 159.587559 51.573508) (end 159.114244 52.716193) (width 2) (layer "F.Cu") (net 5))
 (arc (start 102.554244 177.984193) (mid 102.080929 179.126878) (end 100.938244 179.600193) (width 2) (layer "F.Cu") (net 5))
 (arc (start 148.610244 179.600193) (mid 147.467559 179.126878) (end 146.994244 177.984193) (width 2) (layer "F.Cu") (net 5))
 (arc (start 159.114244 177.984193) (mid 158.640929 179.126878) (end 157.498244 179.600193) (width 2) (layer "F.Cu") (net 5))
 (arc (start 138.914244 52.716193) (mid 138.440929 51.573508) (end 137.298244 51.100193) (width 2) (layer "F.Cu") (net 5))
 (arc (start 169.275 47.425) (mid 169.793076 48.200355) (end 169.975 49.114949) (width 2) (layer "F.Cu") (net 5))
 (arc (start 152.650244 51.100193) (mid 151.507559 51.573508) (end 151.034244 52.716193) (width 2) (layer "F.Cu") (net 5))
 (arc (start 45.994244 177.984193) (mid 45.520929 179.126878) (end 44.378244 179.600193) (width 2) (layer "F.Cu") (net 5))
 (arc (start 75.890244 179.600193) (mid 74.747559 179.126878) (end 74.274244 177.984193) (width 2) (layer "F.Cu") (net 5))
 (arc (start 90.434244 52.716193) (mid 89.960929 51.573508) (end 88.818244 51.100193) (width 2) (layer "F.Cu") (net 5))
 (arc (start 140.530244 179.600193) (mid 139.387559 179.126878) (end 138.914244 177.984193) (width 2) (layer "F.Cu") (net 5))
 (arc (start 163.6 52.513909) (mid 163.52853 52.154604) (end 163.325 51.85) (width 2) (layer "F.Cu") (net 5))
 (arc (start 142.954244 177.984193) (mid 142.480929 179.126878) (end 141.338244 179.600193) (width 2) (layer "F.Cu") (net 5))
 (arc (start 122.754244 52.716193) (mid 122.280929 51.573508) (end 121.138244 51.100193) (width 2) (layer "F.Cu") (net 5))
 (arc (start 37.975 47.1) (mid 40.273097 46.148097) (end 41.225 43.85) (width 2) (layer "F.Cu") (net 5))
 (arc (start 50.034244 52.716193) (mid 49.560929 51.573508) (end 48.418244 51.100193) (width 2) (layer "F.Cu") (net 5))
 (arc (start 88.010244 51.100193) (mid 86.867559 51.573508) (end 86.394244 52.716193) (width 2) (layer "F.Cu") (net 5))
 (arc (start 35.6 167.6) (mid 34.728643 169.703643) (end 32.625 170.575) (width 2) (layer "F.Cu") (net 5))
 (arc (start 96.090244 51.100193) (mid 94.947559 51.573508) (end 94.474244 52.716193) (width 2) (layer "F.Cu") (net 5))
 (arc (start 51.650244 179.600193) (mid 50.507559 179.126878) (end 50.034244 177.984193) (width 2) (layer "F.Cu") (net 5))
 (arc (start 41.954244 52.716193) (mid 41.480929 51.573508) (end 40.338244 51.100193) (width 2) (layer "F.Cu") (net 5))
 (arc (start 130.834244 52.716193) (mid 130.360929 51.573508) (end 129.218244 51.100193) (width 2) (layer "F.Cu") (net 5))
 (arc (start 114.674244 52.716193) (mid 114.200929 51.573508) (end 113.058244 51.100193) (width 2) (layer "F.Cu") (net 5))
 (arc (start 86.394244 177.984193) (mid 85.920929 179.126878) (end 84.778244 179.600193) (width 2) (layer "F.Cu") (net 5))
 (arc (start 134.874244 177.984193) (mid 134.400929 179.126878) (end 133.258244 179.600193) (width 2) (layer "F.Cu") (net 5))
 (arc (start 29.525123 50.374877) (mid 30.484312 48.059189) (end 32.8 47.1) (width 2) (layer "F.Cu") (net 5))
 (arc (start 78.314244 177.984193) (mid 77.840929 179.126878) (end 76.698244 179.600193) (width 2) (layer "F.Cu") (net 5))
 (arc (start 156.690244 179.600193) (mid 155.547559 179.126878) (end 155.074244 177.984193) (width 2) (layer "F.Cu") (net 5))
 (arc (start 155.074244 52.716193) (mid 154.600929 51.573508) (end 153.458244 51.100193) (width 2) (layer "F.Cu") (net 5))
 (arc (start 62.154244 177.984193) (mid 61.680929 179.126878) (end 60.538244 179.600193) (width 2) (layer "F.Cu") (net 5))
 (arc (start 126.794244 177.984193) (mid 126.320929 179.126878) (end 125.178244 179.600193) (width 2) (layer "F.Cu") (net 5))
 (arc (start 94.474244 177.984193) (mid 94.000929 179.126878) (end 92.858244 179.600193) (width 2) (layer "F.Cu") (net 5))
 (arc (start 136.490244 51.100193) (mid 135.347559 51.573508) (end 134.874244 52.716193) (width 2) (layer "F.Cu") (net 5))
 (arc (start 70.234244 177.984193) (mid 69.760929 179.126878) (end 68.618244 179.600193) (width 2) (layer "F.Cu") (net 5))
 (arc (start 47.610244 51.100193) (mid 46.467559 51.573508) (end 45.994244 52.716193) (width 2) (layer "F.Cu") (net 5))
 (arc (start 92.050244 179.600193) (mid 90.907559 179.126878) (end 90.434244 177.984193) (width 2) (layer "F.Cu") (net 5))
 (arc (start 166.275 171.45) (mid 164.383489 170.666511) (end 163.6 168.775) (width 2) (layer "F.Cu") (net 5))
 (arc (start 66.194244 52.716193) (mid 65.720929 51.573508) (end 64.578244 51.100193) (width 2) (layer "F.Cu") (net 5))
 (arc (start 82.354244 52.716193) (mid 81.880929 51.573508) (end 80.738244 51.100193) (width 2) (layer "F.Cu") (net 5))
 (arc (start 31.75 170.575) (mid 30.176774 169.923349) (end 29.525123 168.350123) (width 2) (layer "F.Cu") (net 5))
 (arc (start 74.274244 52.716193) (mid 73.800929 51.573508) (end 72.658244 51.100193) (width 2) (layer "F.Cu") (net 5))
 (arc (start 41.225 42.875) (mid 42.359961 40.134961) (end 45.1 39) (width 2) (layer "F.Cu") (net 5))
 (arc (start 37.249807 51.100193) (mid 36.083217 51.58341) (end 35.6 52.75) (width 2) (layer "F.Cu") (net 5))
 (arc (start 100.130244 179.600193) (mid 98.987559 179.126878) (end 98.514244 177.984193) (width 2) (layer "F.Cu") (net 5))
 (arc (start 112.250244 51.100193) (mid 111.107559 51.573508) (end 110.634244 52.716193) (width 2) (layer "F.Cu") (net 5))
 (arc (start 67.810244 179.600193) (mid 66.667559 179.126878) (end 66.194244 177.984193) (width 2) (layer "F.Cu") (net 5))
 (arc (start 116.290244 179.600193) (mid 115.147559 179.126878) (end 114.674244 177.984193) (width 2) (layer "F.Cu") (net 5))
 (arc (start 144.570244 51.100193) (mid 143.427559 51.573508) (end 142.954244 52.716193) (width 2) (layer "F.Cu") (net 5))
 (arc (start 164.701471 45.05) (mid 166.732647 45.454026) (end 168.454595 46.604595) (width 2) (layer "F.Cu") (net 5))
 (arc (start 106.594244 52.716193) (mid 106.120929 51.573508) (end 104.978244 51.100193) (width 2) (layer "F.Cu") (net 5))
 (arc (start 83.970244 179.600193) (mid 82.827559 179.126878) (end 82.354244 177.984193) (width 2) (layer "F.Cu") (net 5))
 (arc (start 132.450244 179.600193) (mid 131.307559 179.126878) (end 130.834244 177.984193) (width 2) (layer "F.Cu") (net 5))
 (arc (start 124.370244 179.600193) (mid 123.227559 179.126878) (end 122.754244 177.984193) (width 2) (layer "F.Cu") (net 5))
 (arc (start 63.770244 51.100193) (mid 62.627559 51.573508) (end 62.154244 52.716193) (width 2) (layer "F.Cu") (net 5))
 (arc (start 108.210244 179.600193) (mid 107.067559 179.126878) (end 106.594244 177.984193) (width 2) (layer "F.Cu") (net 5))
 (arc (start 58.114244 52.716193) (mid 57.640929 51.573508) (end 56.498244 51.100193) (width 2) (layer "F.Cu") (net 5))
 (segment (start 55.625 46.8) (end 54.8 45.975) (width 0.3) (layer "F.Cu") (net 2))
 (segment (start 55.85 46.8) (end 55.625 46.8) (width 0.3) (layer "F.Cu") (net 2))
 (segment (start 54.8 45.975) (end 53.1 45.975) (width 0.3) (layer "F.Cu") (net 2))
 (via (at 55.85 46.8) (size 0.7) (drill 0.4) (layers "F.Cu" "B.Cu") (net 2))
 (segment (start 55.85 46.8) (end 100.725 46.8) (width 0.3) (layer "B.Cu") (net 2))
 (segment (start 104.9 41.35) (end 106.675 41.35) (width 0.3) (layer "B.Cu") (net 2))
 (segment (start 108.125 39.9) (end 108.125 38.45) (width 0.3) (layer "B.Cu") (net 2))
 (segment (start 104.9 42.625) (end 104.9 41.35) (width 0.3) (layer "B.Cu") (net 2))
 (segment (start 106.675 41.35) (end 108.125 39.9) (width 0.3) (layer "B.Cu") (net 2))
 (segment (start 100.725 46.8) (end 104.9 42.625) (width 0.3) (layer "B.Cu") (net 2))
 (segment (start 112.125 39.025) (end 112.125 38.45) (width 0.3) (layer "F.Cu") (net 4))
 (segment (start 111.05 40.1) (end 112.125 39.025) (width 0.3) (layer "F.Cu") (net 4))
 (segment (start 54.9 47.5) (end 51.125 47.5) (width 0.3) (layer "F.Cu") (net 4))
 (segment (start 109.475 40.1) (end 111.05 40.1) (width 0.3) (layer "F.Cu") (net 4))
 (segment (start 51.125 47.5) (end 49.6 45.975) (width 0.3) (layer "F.Cu") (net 4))
 (segment (start 166.875 167.125) (end 166.875 165.25) (width 0.3) (layer "F.Cu") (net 4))
 (segment (start 167.25 167.5) (end 166.875 167.125) (width 0.3) (layer "F.Cu") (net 4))
 (segment (start 167.775 167.5) (end 167.25 167.5) (width 0.3) (layer "F.Cu") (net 4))
 (via (at 167.775 167.5) (size 0.7) (drill 0.4) (layers "F.Cu" "B.Cu") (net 4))
 (via (at 54.9 47.5) (size 0.7) (drill 0.4) (layers "F.Cu" "B.Cu") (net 4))
 (via (at 109.475 40.1) (size 0.7) (drill 0.4) (layers "F.Cu" "B.Cu") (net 4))
 (segment (start 114.975 41.35) (end 114.975 41.3) (width 0.3) (layer "B.Cu") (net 4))
 (segment (start 114.975 41.35) (end 160.45 41.35) (width 0.3) (layer "B.Cu") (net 4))
 (segment (start 114.975 41.3) (end 112.125 38.45) (width 0.3) (layer "B.Cu") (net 4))
 (segment (start 167.775 167.5) (end 167.775 48.675) (width 0.3) (layer "B.Cu") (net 4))
 (segment (start 109.475 40.1) (end 108.225 41.35) (width 0.3) (layer "B.Cu") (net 4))
 (segment (start 54.9 47.5) (end 102.075 47.5) (width 0.3) (layer "B.Cu") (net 4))
 (segment (start 160.45 41.35) (end 167.775 48.675) (width 0.3) (layer "B.Cu") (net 4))
 (segment (start 102.075 47.5) (end 108.225 41.35) (width 0.3) (layer "B.Cu") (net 4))
 (segment (start 166.875 160.3) (end 166.875 161.75) (width 0.3) (layer "F.Cu") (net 3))
 (via (at 166.875 160.3) (size 0.7) (drill 0.4) (layers "F.Cu" "B.Cu") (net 3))
 (segment (start 113.425 41.35) (end 115.175 43.1) (width 0.3) (layer "B.Cu") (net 3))
 (segment (start 166.875 160.3) (end 166.875 48.95) (width 0.3) (layer "B.Cu") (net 3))
 (segment (start 113.425 41.35) (end 111.6 41.35) (width 0.3) (layer "B.Cu") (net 3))
 (segment (start 111.6 41.35) (end 111.6 39.925) (width 0.3) (layer "B.Cu") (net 3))
 (segment (start 143.85 43.1) (end 161.025 43.1) (width 0.3) (layer "B.Cu") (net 3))
 (segment (start 115.175 43.1) (end 143.85 43.1) (width 0.3) (layer "B.Cu") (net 3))
 (segment (start 166.875 48.95) (end 166.825 48.9) (width 0.3) (layer "B.Cu") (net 3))
 (segment (start 166.825 48.9) (end 165.875 47.95) (width 0.3) (layer "B.Cu") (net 3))
 (segment (start 111.6 39.925) (end 110.125 38.45) (width 0.3) (layer "B.Cu") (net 3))
 (segment (start 161.025 43.1) (end 165.875 47.95) (width 0.3) (layer "B.Cu") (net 3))
 (segment (start 108.65 42.6) (end 107.625 42.6) (width 0.3) (layer "F.Cu") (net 1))
 (segment (start 107.625 42.6) (end 106.125 41.1) (width 0.3) (layer "F.Cu") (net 1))
 (segment (start 106.125 41.1) (end 106.125 38.45) (width 0.3) (layer "F.Cu") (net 1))
 (via (at 108.65 42.6) (size 0.7) (drill 0.4) (layers "F.Cu" "B.Cu") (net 1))
 (segment (start 103.25 41.325) (end 106.125 38.45) (width 0.3) (layer "B.Cu") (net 1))
 (segment (start 109.5 42.35) (end 109.25 42.6) (width 0.3) (layer "B.Cu") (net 1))
 (segment (start 103.25 41.35) (end 103.25 41.325) (width 0.3) (layer "B.Cu") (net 1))
 (segment (start 109.95 41.9) (end 109.5 42.35) (width 0.3) (layer "B.Cu") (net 1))
 (segment (start 109.95 41.35) (end 109.95 41.9) (width 0.3) (layer "B.Cu") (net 1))
 (segment (start 109.25 42.6) (end 108.65 42.6) (width 0.3) (layer "B.Cu") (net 1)))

